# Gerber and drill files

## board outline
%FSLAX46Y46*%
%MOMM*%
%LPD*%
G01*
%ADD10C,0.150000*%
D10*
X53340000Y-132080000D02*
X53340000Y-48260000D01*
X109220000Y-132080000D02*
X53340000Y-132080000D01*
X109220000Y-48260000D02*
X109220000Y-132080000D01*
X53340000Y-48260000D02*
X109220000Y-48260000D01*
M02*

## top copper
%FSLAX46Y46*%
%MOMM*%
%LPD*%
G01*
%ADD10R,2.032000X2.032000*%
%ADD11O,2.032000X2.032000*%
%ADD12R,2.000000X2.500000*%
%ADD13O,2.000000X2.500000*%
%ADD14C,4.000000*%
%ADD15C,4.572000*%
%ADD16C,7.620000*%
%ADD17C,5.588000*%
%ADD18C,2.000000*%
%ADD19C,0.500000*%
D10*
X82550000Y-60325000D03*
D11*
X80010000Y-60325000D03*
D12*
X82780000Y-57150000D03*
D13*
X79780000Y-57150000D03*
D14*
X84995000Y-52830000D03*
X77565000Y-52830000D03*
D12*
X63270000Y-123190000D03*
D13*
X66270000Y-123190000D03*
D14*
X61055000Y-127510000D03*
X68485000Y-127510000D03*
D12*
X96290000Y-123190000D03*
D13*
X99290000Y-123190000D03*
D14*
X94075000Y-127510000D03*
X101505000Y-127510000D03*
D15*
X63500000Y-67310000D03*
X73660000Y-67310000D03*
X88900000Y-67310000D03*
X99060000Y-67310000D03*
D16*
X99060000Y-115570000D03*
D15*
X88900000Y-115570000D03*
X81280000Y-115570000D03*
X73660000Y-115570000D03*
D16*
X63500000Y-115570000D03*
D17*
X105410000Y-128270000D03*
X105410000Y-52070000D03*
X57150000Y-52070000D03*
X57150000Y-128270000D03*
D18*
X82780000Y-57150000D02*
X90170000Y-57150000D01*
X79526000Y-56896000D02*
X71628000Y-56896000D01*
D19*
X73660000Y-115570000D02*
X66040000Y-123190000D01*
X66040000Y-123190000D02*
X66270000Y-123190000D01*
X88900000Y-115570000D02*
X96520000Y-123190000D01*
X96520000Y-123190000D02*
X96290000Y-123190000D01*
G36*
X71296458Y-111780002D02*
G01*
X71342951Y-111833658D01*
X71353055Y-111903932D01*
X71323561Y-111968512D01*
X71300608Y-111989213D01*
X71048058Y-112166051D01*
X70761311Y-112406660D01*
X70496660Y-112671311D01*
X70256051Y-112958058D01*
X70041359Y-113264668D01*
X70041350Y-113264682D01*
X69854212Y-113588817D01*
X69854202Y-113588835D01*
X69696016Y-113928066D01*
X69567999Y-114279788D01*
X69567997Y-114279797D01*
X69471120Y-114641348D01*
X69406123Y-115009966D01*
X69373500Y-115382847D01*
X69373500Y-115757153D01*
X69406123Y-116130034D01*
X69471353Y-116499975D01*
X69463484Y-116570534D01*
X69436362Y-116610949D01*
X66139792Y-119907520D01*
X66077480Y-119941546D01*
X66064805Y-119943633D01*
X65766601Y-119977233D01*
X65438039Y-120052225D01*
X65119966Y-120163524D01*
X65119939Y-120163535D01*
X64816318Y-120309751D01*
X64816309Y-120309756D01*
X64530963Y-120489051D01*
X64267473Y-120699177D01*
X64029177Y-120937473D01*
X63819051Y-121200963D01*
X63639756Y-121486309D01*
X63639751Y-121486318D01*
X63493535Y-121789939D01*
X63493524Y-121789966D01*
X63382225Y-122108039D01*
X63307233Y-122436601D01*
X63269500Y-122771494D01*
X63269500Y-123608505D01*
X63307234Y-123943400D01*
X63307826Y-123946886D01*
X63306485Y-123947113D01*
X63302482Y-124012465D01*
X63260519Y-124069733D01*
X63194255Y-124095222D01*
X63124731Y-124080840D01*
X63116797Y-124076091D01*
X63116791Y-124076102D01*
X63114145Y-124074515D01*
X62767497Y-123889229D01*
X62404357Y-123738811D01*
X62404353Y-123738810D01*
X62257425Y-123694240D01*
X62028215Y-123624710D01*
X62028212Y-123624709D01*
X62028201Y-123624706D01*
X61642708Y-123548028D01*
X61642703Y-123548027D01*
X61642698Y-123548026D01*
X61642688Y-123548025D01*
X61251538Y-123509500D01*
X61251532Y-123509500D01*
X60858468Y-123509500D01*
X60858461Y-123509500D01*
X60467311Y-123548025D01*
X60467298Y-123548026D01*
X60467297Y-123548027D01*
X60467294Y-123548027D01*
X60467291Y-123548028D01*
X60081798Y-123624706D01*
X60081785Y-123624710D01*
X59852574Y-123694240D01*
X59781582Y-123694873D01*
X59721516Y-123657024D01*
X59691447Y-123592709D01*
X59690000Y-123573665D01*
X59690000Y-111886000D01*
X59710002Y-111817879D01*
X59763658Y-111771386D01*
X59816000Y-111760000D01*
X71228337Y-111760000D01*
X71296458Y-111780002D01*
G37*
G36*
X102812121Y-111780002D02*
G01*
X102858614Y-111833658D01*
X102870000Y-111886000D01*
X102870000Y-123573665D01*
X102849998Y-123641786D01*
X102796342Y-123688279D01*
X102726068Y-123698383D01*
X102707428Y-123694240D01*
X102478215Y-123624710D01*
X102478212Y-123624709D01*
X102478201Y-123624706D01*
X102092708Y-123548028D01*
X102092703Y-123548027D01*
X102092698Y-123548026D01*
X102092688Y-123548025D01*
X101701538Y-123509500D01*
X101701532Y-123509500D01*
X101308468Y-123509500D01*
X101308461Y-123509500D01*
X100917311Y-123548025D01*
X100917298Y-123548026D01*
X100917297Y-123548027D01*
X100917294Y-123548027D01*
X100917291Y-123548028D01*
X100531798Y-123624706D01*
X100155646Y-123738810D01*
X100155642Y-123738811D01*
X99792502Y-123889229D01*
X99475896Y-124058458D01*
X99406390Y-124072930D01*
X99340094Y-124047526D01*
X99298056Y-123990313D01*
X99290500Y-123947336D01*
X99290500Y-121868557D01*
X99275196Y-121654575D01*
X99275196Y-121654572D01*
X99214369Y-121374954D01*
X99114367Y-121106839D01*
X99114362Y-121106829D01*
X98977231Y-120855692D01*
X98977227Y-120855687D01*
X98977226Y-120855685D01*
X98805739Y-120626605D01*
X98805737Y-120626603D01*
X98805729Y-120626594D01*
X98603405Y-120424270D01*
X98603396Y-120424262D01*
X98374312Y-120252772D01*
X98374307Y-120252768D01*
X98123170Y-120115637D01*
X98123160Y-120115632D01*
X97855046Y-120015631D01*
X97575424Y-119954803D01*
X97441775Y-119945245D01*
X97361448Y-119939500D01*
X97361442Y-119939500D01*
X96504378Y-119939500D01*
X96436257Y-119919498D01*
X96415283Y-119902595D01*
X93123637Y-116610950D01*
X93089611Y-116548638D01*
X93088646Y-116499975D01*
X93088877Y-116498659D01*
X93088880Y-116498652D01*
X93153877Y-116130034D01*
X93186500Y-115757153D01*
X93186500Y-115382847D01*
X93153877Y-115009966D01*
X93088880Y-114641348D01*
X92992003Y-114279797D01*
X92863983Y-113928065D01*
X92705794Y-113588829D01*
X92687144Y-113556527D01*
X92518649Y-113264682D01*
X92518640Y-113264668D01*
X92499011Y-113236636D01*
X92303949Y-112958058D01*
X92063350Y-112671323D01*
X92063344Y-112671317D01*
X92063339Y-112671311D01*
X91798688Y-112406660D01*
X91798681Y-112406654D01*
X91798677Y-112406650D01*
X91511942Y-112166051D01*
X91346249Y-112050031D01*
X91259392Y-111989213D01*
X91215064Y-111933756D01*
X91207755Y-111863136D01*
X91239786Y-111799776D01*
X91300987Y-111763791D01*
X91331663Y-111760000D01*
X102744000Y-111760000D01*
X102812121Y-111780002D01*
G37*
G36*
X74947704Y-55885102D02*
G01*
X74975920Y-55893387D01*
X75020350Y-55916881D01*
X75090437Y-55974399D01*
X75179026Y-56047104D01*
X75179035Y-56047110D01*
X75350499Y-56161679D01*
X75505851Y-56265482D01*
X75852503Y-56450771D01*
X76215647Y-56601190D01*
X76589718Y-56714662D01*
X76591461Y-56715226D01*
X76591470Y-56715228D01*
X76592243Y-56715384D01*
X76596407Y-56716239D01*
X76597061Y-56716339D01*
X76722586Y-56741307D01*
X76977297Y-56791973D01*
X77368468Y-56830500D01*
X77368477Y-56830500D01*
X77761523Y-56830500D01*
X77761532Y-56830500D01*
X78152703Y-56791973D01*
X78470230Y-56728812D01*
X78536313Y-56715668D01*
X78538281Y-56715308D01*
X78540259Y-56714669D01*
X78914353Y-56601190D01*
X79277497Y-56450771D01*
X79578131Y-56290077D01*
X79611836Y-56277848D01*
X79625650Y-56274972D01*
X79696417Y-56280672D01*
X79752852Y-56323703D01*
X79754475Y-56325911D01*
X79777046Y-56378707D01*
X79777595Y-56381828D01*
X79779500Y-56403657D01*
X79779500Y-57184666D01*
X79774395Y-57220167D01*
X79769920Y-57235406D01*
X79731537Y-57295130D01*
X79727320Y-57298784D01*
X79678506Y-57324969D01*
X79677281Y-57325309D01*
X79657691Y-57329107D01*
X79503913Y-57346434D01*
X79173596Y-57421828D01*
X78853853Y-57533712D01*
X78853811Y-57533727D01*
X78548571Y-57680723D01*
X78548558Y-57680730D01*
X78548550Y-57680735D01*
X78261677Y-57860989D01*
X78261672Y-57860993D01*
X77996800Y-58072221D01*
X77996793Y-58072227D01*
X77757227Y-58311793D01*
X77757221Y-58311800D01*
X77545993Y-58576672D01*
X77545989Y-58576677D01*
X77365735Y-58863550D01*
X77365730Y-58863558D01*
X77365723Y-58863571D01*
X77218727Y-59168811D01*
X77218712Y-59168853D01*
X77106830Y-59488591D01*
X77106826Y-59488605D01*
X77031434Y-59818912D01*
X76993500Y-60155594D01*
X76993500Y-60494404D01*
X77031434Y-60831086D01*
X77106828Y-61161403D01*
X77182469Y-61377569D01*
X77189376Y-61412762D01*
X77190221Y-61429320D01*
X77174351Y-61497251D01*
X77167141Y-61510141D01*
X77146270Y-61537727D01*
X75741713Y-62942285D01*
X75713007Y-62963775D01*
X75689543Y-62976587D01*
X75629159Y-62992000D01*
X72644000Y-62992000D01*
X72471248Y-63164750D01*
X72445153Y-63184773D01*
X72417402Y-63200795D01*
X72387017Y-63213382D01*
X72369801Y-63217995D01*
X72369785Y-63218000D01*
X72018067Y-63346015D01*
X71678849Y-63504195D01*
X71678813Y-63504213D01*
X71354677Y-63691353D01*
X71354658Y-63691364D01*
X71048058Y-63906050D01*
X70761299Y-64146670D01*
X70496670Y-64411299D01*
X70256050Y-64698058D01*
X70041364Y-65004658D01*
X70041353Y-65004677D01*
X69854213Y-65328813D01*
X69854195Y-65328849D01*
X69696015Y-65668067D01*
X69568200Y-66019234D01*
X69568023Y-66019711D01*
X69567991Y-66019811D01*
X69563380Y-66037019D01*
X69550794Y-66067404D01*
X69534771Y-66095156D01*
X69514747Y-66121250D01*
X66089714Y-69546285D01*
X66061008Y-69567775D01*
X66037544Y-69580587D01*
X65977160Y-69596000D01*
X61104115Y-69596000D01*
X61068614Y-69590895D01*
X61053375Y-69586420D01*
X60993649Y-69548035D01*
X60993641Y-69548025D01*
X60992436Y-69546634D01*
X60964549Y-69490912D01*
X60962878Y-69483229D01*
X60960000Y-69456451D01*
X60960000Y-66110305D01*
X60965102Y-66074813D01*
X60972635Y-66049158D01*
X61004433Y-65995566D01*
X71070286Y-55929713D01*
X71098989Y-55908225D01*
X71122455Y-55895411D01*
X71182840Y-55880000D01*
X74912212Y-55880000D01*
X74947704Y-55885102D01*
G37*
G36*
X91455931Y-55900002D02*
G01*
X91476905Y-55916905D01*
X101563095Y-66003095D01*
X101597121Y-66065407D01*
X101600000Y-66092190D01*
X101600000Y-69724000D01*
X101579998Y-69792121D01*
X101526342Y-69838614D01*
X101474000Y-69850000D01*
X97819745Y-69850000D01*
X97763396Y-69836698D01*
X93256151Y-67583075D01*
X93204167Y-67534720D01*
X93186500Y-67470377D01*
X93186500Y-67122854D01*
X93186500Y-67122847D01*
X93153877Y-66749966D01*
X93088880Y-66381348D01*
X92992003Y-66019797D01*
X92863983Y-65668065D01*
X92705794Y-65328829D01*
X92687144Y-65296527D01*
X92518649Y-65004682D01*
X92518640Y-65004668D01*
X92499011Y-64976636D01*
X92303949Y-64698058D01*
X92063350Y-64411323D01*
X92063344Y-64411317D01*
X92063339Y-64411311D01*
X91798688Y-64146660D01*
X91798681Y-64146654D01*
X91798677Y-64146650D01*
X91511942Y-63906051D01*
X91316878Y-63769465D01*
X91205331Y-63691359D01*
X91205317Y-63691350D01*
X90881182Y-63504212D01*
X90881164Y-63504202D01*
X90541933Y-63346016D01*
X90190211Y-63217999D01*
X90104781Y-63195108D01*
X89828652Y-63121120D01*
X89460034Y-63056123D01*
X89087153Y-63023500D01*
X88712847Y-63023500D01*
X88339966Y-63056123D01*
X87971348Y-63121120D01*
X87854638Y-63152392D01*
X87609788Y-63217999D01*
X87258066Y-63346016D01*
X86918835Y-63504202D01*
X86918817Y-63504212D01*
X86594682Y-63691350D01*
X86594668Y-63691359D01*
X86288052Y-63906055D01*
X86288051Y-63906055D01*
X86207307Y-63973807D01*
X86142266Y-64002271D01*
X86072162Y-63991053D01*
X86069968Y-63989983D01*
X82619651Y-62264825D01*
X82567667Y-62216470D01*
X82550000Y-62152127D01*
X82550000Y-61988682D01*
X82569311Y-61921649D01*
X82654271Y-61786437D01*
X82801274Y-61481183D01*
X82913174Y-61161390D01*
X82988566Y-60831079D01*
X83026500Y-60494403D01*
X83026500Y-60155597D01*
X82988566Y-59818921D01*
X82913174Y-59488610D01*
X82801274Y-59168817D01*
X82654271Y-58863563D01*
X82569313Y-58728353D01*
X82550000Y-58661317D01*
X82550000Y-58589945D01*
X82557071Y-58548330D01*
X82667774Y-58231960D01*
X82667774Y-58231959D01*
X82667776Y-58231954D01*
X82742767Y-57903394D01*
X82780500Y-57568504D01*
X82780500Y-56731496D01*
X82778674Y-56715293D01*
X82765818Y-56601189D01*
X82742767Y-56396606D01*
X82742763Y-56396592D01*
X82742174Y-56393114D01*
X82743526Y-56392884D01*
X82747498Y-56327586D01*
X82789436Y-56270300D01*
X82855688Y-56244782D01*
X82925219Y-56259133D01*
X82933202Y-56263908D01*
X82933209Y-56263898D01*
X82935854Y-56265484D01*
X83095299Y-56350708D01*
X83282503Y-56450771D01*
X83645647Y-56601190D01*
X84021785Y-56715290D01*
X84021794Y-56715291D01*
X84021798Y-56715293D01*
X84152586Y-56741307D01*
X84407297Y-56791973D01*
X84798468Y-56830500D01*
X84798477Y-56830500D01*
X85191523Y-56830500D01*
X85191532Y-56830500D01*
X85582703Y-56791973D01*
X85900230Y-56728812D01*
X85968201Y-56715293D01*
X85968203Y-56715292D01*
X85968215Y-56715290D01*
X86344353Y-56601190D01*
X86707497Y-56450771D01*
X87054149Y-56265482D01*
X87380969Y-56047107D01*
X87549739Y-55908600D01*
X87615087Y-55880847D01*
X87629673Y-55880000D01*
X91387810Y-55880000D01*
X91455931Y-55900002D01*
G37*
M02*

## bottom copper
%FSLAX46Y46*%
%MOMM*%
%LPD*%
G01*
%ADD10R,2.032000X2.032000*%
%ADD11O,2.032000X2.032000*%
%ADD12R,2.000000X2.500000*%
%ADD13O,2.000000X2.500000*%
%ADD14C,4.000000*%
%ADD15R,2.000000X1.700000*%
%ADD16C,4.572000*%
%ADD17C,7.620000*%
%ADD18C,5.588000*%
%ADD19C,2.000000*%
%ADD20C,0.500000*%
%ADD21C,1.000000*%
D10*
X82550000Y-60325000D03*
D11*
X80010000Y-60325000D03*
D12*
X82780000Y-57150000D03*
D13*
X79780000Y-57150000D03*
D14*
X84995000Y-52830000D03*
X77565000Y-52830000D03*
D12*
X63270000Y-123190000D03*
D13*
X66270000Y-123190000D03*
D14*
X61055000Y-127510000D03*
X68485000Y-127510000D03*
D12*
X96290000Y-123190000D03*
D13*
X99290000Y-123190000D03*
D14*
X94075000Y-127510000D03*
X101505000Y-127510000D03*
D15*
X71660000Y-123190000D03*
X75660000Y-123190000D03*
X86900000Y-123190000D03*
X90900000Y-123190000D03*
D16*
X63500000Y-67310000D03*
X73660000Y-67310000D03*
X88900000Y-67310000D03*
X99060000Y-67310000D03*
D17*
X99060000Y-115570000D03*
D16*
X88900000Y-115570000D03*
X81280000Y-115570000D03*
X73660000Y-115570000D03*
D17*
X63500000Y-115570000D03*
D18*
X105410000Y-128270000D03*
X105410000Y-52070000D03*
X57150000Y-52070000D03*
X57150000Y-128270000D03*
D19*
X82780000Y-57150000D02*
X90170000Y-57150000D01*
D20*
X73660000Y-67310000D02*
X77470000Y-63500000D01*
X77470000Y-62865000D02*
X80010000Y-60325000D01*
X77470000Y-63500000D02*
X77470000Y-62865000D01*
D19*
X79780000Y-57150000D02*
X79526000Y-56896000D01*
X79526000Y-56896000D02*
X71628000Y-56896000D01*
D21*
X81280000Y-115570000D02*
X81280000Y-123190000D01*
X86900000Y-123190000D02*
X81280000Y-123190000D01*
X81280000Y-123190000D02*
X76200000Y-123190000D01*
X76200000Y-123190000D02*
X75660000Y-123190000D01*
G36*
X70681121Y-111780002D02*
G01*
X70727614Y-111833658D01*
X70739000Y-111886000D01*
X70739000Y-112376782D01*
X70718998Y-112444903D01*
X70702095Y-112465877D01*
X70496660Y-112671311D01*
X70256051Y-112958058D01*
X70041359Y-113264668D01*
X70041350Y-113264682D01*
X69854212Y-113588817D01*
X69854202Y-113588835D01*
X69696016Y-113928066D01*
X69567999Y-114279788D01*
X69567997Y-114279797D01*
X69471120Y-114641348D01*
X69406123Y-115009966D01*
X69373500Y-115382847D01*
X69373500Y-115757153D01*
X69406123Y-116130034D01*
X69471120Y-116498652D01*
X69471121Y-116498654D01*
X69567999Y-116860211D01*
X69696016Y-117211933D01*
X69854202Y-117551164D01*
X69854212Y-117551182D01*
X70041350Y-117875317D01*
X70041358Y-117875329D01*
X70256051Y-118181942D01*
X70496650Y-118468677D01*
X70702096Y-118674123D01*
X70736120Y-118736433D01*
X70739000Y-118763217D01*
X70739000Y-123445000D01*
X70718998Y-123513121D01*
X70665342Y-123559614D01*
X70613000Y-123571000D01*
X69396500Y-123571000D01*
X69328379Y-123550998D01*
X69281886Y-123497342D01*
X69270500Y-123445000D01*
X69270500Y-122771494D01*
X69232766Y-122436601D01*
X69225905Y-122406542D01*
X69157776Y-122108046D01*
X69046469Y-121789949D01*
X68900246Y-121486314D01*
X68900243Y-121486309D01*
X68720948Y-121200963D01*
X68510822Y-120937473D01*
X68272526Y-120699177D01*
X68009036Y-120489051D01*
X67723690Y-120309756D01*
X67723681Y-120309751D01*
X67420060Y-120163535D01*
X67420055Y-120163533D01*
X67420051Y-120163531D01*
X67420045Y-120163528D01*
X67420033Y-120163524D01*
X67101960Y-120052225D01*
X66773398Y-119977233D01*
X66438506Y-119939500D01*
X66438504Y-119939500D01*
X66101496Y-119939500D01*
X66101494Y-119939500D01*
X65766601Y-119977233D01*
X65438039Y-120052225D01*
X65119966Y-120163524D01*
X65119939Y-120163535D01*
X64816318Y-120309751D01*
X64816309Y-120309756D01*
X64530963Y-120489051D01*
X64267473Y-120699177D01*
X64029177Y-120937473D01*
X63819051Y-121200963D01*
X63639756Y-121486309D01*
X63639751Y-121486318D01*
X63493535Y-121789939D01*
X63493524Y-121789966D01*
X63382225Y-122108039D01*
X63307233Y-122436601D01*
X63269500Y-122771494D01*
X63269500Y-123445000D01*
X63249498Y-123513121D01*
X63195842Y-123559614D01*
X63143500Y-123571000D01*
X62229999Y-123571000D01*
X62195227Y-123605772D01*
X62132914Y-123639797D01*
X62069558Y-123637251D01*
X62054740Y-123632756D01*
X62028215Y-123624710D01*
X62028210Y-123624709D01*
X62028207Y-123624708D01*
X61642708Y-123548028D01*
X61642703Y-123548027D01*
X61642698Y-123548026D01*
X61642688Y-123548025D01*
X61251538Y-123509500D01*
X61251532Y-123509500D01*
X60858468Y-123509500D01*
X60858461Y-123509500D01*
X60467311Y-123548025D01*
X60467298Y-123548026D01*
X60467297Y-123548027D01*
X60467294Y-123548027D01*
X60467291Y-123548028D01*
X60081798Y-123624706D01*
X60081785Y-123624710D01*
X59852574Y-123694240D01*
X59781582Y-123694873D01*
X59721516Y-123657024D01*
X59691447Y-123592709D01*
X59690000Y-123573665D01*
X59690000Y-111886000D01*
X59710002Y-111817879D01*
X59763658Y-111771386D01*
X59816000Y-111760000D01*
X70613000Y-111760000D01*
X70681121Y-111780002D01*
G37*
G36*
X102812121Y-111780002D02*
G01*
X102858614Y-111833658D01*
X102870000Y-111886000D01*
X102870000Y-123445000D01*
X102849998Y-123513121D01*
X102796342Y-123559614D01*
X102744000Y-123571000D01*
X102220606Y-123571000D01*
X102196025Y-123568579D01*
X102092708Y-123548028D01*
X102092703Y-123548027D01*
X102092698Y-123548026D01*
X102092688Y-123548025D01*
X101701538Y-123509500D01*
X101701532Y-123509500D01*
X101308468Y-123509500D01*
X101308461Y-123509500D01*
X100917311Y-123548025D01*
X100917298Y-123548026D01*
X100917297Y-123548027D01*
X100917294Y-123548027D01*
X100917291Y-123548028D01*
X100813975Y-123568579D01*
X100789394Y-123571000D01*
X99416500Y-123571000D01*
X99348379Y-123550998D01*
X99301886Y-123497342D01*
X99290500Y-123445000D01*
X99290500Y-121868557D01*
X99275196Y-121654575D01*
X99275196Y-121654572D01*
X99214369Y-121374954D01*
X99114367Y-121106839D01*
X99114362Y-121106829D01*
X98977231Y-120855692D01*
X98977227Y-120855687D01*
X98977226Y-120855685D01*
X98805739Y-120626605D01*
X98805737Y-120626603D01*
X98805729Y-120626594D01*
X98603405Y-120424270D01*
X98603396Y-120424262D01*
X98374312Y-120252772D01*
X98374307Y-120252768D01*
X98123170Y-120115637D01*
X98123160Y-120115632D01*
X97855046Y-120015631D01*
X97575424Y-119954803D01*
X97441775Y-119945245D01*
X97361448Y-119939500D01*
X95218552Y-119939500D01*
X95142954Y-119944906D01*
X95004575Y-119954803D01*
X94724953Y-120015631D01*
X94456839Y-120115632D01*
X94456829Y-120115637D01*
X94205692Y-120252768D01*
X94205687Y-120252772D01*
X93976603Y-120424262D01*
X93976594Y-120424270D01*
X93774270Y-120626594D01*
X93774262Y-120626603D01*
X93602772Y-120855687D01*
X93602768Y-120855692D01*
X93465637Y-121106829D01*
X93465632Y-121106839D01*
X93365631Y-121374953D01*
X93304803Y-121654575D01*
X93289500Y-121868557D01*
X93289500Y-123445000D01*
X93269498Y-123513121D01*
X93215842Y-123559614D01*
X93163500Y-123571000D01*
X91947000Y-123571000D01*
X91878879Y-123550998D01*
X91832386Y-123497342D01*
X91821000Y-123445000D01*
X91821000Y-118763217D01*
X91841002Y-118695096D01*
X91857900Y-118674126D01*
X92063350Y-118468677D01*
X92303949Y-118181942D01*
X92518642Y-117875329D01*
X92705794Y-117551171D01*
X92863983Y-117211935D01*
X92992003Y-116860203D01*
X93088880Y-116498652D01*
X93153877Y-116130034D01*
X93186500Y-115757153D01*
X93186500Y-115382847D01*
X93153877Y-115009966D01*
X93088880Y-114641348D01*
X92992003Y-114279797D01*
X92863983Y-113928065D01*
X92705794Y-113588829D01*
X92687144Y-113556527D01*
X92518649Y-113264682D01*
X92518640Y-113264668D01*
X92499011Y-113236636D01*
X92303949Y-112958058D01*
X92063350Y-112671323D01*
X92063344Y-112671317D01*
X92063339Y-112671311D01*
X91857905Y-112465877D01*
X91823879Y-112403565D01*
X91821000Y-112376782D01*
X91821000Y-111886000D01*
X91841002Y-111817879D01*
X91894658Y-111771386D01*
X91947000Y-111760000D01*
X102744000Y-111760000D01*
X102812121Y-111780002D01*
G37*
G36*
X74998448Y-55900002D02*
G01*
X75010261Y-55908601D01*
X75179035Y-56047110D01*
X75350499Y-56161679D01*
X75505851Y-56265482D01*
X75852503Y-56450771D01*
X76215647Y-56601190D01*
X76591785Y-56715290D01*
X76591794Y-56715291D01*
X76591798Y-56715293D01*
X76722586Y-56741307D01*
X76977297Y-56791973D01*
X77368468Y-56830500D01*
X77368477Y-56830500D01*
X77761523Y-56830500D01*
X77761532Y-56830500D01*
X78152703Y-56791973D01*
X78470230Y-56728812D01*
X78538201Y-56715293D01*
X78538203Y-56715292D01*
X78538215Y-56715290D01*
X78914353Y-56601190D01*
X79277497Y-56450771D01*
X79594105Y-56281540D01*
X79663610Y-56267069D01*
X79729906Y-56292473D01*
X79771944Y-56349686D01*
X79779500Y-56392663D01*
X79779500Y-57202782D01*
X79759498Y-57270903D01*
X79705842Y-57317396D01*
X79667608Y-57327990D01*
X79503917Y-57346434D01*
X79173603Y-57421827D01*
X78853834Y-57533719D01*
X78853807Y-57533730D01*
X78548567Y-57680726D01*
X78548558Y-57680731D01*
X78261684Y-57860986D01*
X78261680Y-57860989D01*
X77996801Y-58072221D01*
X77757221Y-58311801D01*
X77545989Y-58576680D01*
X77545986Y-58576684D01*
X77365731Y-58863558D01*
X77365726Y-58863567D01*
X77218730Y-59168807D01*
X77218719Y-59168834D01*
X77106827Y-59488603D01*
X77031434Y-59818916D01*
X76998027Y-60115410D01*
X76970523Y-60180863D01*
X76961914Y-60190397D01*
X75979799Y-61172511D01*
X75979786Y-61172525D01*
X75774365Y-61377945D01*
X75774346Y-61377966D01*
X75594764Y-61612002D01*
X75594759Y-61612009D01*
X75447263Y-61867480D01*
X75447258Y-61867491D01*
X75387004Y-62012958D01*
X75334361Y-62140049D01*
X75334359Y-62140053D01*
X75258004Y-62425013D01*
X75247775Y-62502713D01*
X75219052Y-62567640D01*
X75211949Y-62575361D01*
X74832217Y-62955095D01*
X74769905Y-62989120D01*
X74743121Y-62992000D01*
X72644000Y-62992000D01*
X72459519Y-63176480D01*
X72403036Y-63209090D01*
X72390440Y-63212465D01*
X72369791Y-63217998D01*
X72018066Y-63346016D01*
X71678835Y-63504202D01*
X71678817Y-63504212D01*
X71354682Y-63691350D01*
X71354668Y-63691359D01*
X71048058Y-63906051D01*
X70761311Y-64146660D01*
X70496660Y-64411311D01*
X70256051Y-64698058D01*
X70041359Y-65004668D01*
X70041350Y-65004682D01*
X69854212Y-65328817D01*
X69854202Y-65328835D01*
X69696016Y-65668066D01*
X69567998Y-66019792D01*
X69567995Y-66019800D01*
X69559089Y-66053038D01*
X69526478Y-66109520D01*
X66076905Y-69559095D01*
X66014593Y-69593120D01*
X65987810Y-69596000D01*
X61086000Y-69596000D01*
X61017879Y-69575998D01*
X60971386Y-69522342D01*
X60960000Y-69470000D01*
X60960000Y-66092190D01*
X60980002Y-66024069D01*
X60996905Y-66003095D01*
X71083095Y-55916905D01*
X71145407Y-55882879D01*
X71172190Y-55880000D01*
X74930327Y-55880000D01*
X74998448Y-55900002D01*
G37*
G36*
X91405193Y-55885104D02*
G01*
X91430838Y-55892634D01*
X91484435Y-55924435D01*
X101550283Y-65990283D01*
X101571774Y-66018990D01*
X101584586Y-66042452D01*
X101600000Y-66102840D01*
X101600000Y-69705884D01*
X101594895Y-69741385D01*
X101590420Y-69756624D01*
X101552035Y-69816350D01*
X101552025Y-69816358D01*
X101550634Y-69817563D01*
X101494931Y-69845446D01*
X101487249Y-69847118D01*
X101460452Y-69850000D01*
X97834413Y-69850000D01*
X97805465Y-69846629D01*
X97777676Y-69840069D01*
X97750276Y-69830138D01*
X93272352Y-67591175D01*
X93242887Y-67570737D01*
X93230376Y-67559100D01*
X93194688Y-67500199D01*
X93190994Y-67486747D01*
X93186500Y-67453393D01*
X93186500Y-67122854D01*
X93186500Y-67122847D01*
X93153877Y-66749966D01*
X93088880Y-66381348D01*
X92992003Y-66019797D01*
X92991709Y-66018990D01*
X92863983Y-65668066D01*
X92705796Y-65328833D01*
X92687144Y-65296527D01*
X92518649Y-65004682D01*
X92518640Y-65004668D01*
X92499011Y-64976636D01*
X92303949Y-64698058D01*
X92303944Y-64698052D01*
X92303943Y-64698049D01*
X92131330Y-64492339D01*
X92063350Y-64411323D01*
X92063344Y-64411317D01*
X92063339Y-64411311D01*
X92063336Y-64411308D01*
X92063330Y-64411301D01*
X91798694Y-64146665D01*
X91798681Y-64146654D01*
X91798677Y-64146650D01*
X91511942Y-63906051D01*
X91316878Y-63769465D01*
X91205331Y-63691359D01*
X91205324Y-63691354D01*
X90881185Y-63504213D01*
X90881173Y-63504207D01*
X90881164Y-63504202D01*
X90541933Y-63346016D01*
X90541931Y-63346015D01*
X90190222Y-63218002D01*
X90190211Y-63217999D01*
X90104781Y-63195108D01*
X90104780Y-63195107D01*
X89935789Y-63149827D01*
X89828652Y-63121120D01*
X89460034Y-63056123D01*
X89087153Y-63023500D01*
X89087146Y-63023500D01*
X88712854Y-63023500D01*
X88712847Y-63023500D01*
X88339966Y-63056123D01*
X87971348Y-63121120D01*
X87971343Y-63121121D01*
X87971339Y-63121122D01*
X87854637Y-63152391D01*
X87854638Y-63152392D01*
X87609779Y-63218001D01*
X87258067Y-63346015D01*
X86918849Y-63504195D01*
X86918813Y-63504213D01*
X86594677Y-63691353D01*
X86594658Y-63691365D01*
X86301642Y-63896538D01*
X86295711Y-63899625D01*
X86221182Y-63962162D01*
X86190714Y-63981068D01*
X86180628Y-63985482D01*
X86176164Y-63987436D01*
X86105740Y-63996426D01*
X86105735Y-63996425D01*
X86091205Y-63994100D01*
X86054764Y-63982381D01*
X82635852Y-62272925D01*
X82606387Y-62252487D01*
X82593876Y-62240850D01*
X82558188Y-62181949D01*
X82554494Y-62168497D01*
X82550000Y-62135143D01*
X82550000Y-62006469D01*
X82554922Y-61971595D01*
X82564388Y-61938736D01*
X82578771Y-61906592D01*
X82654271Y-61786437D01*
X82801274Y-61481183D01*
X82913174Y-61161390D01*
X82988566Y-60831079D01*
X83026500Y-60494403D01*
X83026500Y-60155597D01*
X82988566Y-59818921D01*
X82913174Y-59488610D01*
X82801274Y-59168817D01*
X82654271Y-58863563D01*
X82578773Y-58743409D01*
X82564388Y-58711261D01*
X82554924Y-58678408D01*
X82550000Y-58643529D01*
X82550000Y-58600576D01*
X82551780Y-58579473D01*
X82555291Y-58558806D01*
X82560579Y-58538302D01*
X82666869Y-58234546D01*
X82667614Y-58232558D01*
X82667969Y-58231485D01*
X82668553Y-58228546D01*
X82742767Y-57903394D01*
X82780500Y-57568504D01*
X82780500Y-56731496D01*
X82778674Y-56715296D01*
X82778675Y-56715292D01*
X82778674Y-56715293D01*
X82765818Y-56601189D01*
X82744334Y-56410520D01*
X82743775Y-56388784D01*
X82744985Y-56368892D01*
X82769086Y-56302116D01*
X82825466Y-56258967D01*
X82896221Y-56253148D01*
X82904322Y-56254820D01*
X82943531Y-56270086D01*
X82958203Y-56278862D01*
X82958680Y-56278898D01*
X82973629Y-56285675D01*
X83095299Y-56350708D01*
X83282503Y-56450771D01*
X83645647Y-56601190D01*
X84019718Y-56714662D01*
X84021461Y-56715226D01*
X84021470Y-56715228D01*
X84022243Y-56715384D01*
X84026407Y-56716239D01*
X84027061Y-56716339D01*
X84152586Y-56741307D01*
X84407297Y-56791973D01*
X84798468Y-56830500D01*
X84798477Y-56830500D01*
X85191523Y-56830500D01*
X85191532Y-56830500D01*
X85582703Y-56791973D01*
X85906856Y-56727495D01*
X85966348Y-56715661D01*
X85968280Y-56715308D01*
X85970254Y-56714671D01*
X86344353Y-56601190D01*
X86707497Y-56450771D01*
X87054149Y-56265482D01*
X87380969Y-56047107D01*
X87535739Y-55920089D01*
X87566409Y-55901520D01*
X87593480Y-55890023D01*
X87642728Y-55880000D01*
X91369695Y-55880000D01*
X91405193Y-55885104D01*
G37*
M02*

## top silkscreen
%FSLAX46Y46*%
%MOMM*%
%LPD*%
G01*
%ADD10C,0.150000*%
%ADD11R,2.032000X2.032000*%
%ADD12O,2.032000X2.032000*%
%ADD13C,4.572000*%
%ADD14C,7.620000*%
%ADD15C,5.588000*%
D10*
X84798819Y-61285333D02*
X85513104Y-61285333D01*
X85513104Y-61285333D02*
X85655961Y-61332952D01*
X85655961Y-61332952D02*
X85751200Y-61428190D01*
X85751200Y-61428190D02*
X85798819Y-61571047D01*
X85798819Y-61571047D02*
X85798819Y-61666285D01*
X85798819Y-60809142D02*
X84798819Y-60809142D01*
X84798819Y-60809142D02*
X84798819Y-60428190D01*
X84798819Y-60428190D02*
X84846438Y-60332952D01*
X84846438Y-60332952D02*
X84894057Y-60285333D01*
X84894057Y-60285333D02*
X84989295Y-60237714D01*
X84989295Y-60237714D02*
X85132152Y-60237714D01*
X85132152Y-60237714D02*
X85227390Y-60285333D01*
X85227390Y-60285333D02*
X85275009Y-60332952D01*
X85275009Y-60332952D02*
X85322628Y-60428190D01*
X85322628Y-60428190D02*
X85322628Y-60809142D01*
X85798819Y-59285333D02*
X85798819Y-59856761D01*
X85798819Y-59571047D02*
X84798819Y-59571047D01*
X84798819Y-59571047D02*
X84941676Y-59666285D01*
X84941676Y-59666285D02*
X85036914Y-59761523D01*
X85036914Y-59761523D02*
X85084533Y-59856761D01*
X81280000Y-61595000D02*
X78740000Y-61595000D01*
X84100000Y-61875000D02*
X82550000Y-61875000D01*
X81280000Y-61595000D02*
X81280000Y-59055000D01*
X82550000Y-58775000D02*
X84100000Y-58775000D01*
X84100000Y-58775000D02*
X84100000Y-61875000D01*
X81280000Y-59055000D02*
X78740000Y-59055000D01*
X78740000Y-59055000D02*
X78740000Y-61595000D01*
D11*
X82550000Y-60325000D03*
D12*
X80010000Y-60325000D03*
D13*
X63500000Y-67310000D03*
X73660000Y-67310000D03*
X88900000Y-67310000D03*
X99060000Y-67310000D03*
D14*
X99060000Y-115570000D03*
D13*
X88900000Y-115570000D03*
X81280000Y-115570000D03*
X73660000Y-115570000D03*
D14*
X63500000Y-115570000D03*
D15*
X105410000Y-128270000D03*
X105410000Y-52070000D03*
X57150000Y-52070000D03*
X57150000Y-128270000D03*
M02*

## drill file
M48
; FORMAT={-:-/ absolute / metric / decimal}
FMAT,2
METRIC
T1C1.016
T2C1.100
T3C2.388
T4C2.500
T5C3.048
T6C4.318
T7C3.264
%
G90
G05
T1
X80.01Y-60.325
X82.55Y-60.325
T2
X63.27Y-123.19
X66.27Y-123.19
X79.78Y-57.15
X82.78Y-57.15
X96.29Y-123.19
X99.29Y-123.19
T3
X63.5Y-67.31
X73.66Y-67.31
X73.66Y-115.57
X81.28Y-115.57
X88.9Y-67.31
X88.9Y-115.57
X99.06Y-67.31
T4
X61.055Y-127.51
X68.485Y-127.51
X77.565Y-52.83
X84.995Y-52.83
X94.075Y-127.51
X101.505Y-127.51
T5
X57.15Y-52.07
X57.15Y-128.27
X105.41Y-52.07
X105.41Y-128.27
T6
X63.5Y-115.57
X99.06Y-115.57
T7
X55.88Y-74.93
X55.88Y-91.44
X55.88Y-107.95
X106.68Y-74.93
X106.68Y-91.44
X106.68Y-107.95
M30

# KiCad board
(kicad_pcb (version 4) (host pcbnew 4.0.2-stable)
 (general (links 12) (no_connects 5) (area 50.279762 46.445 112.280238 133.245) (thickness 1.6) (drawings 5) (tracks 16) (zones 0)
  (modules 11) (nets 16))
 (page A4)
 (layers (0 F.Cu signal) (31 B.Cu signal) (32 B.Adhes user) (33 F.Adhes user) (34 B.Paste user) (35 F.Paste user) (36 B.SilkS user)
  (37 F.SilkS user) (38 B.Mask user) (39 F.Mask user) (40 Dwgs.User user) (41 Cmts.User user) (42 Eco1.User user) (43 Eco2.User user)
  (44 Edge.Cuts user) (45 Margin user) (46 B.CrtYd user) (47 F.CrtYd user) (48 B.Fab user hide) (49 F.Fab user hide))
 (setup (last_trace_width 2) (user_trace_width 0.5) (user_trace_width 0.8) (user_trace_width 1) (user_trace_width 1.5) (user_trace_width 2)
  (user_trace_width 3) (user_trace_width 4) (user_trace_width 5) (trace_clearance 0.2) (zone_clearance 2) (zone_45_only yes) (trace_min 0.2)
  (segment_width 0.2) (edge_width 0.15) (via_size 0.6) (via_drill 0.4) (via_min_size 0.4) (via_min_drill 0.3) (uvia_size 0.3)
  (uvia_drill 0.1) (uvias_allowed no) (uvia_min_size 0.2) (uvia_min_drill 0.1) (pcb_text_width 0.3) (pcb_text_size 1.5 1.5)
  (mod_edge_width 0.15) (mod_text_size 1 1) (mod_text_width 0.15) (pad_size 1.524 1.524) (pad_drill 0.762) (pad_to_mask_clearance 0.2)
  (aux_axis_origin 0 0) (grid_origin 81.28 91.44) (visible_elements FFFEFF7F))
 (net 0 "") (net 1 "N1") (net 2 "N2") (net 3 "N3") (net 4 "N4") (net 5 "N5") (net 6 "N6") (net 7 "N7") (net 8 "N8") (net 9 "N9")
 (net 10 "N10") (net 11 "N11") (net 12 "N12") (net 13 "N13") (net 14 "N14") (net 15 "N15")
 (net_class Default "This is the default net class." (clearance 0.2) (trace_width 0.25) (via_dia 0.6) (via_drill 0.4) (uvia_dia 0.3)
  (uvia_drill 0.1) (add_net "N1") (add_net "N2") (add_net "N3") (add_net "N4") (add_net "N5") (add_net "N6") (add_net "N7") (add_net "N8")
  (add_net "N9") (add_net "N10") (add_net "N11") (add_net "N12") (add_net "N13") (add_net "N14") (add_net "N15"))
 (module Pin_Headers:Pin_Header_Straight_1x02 (layer F.Cu) (at 82.55 60.325 270)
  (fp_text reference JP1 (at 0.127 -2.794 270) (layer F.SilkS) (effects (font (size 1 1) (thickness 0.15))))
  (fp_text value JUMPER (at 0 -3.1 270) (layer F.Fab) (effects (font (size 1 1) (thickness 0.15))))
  (fp_line (start 1.27 1.27) (end 1.27 3.81) (layer F.SilkS) (width 0.15))
  (fp_line (start 1.55 -1.55) (end 1.55 0) (layer F.SilkS) (width 0.15))
  (fp_line (start 1.27 1.27) (end -1.27 1.27) (layer F.SilkS) (width 0.15))
  (fp_line (start -1.55 0) (end -1.55 -1.55) (layer F.SilkS) (width 0.15))
  (fp_line (start -1.55 -1.55) (end 1.55 -1.55) (layer F.SilkS) (width 0.15))
  (fp_line (start -1.27 1.27) (end -1.27 3.81) (layer F.SilkS) (width 0.15))
  (fp_line (start -1.27 3.81) (end 1.27 3.81) (layer F.SilkS) (width 0.15))
  (pad 1 thru_hole rect (at 0 0 270) (size 2.032 2.032) (drill 1.016) (layers *.Cu *.Mask F.SilkS) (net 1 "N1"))
  (pad 2 thru_hole oval (at 0 2.54 270) (size 2.032 2.032) (drill 1.016) (layers *.Cu *.Mask F.SilkS) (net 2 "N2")))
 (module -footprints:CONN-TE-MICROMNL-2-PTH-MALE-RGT (layer B.Cu) (at 81.28 57.15)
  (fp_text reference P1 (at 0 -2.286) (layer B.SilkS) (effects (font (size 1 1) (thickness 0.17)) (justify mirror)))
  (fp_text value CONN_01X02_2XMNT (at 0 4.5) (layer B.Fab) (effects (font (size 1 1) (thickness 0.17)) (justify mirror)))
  (pad 1 thru_hole rect (at 1.5 0) (size 2 2.5) (drill 1.1) (layers *.Cu *.Mask B.SilkS) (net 1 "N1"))
  (pad 2 thru_hole oval (at -1.5 0) (size 2 2.5) (drill 1.1) (layers *.Cu *.Mask B.SilkS) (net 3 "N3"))
  (pad M1 thru_hole circle (at 3.715 -4.32) (size 4 4) (drill 2.5) (layers *.Cu *.Mask B.SilkS) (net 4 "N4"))
  (pad M2 thru_hole circle (at -3.715 -4.32) (size 4 4) (drill 2.5) (layers *.Cu *.Mask B.SilkS) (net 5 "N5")))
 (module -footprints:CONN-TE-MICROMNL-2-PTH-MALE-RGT (layer B.Cu) (at 64.77 123.19 180)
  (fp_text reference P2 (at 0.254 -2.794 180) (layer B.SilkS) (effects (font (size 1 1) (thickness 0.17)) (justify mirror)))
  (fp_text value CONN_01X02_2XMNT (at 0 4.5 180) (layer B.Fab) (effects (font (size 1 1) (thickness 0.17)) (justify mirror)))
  (pad 1 thru_hole rect (at 1.5 0 180) (size 2 2.5) (drill 1.1) (layers *.Cu *.Mask B.SilkS) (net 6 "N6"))
  (pad 2 thru_hole oval (at -1.5 0 180) (size 2 2.5) (drill 1.1) (layers *.Cu *.Mask B.SilkS) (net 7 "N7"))
  (pad M1 thru_hole circle (at 3.715 -4.32 180) (size 4 4) (drill 2.5) (layers *.Cu *.Mask B.SilkS) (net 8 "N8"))
  (pad M2 thru_hole circle (at -3.715 -4.32 180) (size 4 4) (drill 2.5) (layers *.Cu *.Mask B.SilkS) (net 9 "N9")))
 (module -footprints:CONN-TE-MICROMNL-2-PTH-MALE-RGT (layer B.Cu) (at 97.79 123.19 180)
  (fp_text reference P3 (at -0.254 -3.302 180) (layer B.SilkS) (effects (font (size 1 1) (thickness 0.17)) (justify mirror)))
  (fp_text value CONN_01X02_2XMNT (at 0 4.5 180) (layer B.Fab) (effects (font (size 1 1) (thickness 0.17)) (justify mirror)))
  (pad 1 thru_hole rect (at 1.5 0 180) (size 2 2.5) (drill 1.1) (layers *.Cu *.Mask B.SilkS) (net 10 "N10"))
  (pad 2 thru_hole oval (at -1.5 0 180) (size 2 2.5) (drill 1.1) (layers *.Cu *.Mask B.SilkS) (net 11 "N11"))
  (pad M1 thru_hole circle (at 3.715 -4.32 180) (size 4 4) (drill 2.5) (layers *.Cu *.Mask B.SilkS) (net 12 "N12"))
  (pad M2 thru_hole circle (at -3.715 -4.32 180) (size 4 4) (drill 2.5) (layers *.Cu *.Mask B.SilkS) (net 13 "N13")))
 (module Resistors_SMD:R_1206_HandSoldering (layer B.Cu) (at 73.66 123.19)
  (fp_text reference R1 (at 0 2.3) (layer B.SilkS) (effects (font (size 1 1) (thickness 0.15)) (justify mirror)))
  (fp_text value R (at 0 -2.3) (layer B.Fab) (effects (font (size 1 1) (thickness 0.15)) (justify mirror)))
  (pad 1 smd rect (at -2 0) (size 2 1.7) (layers B.Cu B.Paste B.Mask) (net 6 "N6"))
  (pad 2 smd rect (at 2 0) (size 2 1.7) (layers B.Cu B.Paste B.Mask) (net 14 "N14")))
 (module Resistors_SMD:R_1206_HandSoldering (layer B.Cu) (at 88.9 123.19)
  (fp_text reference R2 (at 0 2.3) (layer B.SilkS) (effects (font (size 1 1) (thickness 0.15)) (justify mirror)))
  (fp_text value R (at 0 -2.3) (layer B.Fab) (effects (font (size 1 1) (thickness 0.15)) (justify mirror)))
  (pad 1 smd rect (at -2 0) (size 2 1.7) (layers B.Cu B.Paste B.Mask) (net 14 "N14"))
  (pad 2 smd rect (at 2 0) (size 2 1.7) (layers B.Cu B.Paste B.Mask) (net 11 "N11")))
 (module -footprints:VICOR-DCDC (layer F.Cu) (at 81.28 91.44)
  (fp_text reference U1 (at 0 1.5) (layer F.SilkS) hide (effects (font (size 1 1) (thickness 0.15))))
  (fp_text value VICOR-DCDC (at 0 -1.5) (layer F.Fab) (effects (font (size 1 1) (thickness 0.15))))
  (pad 1 thru_hole circle (at -17.78 -24.13) (size 4.572 4.572) (drill 2.3876) (layers *.Cu *.Mask F.SilkS) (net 3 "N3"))
  (pad 2 thru_hole circle (at -7.62 -24.13) (size 4.572 4.572) (drill 2.3876) (layers *.Cu *.Mask F.SilkS) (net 2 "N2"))
  (pad 3 thru_hole circle (at 7.62 -24.13) (size 4.572 4.572) (drill 2.3876) (layers *.Cu *.Mask F.SilkS) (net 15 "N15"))
  (pad 4 thru_hole circle (at 17.78 -24.13) (size 4.572 4.572) (drill 2.3876) (layers *.Cu *.Mask F.SilkS) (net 1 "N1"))
  (pad 5 thru_hole circle (at 17.78 24.13) (size 7.62 7.62) (drill 4.318) (layers *.Cu *.Mask F.SilkS) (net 11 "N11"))
  (pad 6 thru_hole circle (at 7.62 24.13) (size 4.572 4.572) (drill 2.3876) (layers *.Cu *.Mask F.SilkS) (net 10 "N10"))
  (pad 7 thru_hole circle (at 0 24.13) (size 4.572 4.572) (drill 2.3876) (layers *.Cu *.Mask F.SilkS) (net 14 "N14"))
  (pad 8 thru_hole circle (at -7.62 24.13) (size 4.572 4.572) (drill 2.3876) (layers *.Cu *.Mask F.SilkS) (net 7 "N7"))
  (pad 9 thru_hole circle (at -17.78 24.13) (size 7.62 7.62) (drill 4.318) (layers *.Cu *.Mask F.SilkS) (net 6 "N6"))
  (pad "" np_thru_hole circle (at -25.4 0) (size 3.2639 3.2639) (drill 3.2639) (layers *.Cu))
  (pad "" np_thru_hole circle (at 25.4 0) (size 3.2639 3.2639) (drill 3.2639) (layers *.Cu))
  (pad "" np_thru_hole circle (at 25.4 -16.51) (size 3.2639 3.2639) (drill 3.2639) (layers *.Cu))
  (pad "" np_thru_hole circle (at 25.4 16.51) (size 3.2639 3.2639) (drill 3.2639) (layers *.Cu))
  (pad "" np_thru_hole circle (at -25.4 16.51) (size 3.2639 3.2639) (drill 3.2639) (layers *.Cu))
  (pad "" np_thru_hole circle (at -25.4 -16.51) (size 3.2639 3.2639) (drill 3.2639) (layers *.Cu)))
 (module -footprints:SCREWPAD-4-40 (layer F.Cu) (at 105.41 128.27)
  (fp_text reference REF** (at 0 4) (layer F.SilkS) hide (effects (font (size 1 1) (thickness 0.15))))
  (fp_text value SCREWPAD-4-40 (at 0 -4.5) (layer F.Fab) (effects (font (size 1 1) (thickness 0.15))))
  (pad 1 thru_hole circle (at 0 0) (size 5.588 5.588) (drill 3.048) (layers *.Cu *.Mask F.SilkS)))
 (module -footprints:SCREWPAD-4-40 (layer F.Cu) (at 105.41 52.07)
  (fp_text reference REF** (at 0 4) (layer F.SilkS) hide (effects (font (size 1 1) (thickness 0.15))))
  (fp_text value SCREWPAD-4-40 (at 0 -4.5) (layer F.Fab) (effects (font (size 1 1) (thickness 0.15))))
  (pad 1 thru_hole circle (at 0 0) (size 5.588 5.588) (drill 3.048) (layers *.Cu *.Mask F.SilkS)))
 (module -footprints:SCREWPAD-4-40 (layer F.Cu) (at 57.15 52.07)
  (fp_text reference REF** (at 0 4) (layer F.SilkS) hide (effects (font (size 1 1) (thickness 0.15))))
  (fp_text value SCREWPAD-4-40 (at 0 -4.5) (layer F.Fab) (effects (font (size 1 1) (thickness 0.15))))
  (pad 1 thru_hole circle (at 0 0) (size 5.588 5.588) (drill 3.048) (layers *.Cu *.Mask F.SilkS)))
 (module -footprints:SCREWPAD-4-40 (layer F.Cu) (at 57.15 128.27)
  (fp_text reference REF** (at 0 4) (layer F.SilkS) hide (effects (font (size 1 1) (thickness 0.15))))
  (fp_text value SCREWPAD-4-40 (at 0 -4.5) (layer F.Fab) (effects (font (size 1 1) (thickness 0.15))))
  (pad 1 thru_hole circle (at 0 0) (size 5.588 5.588) (drill 3.048) (layers *.Cu *.Mask F.SilkS)))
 (gr_line (start 53.34 132.08) (end 53.34 48.26) (angle 90) (layer Edge.Cuts) (width 0.15))
 (gr_line (start 109.22 132.08) (end 53.34 132.08) (angle 90) (layer Edge.Cuts) (width 0.15))
 (gr_line (start 109.22 48.26) (end 109.22 132.08) (angle 90) (layer Edge.Cuts) (width 0.15))
 (gr_line (start 53.34 48.26) (end 109.22 48.26) (angle 90) (layer Edge.Cuts) (width 0.15))
 (segment (start 82.78 57.15) (end 90.17 57.15) (width 2) (layer F.Cu) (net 1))
 (segment (start 82.78 57.15) (end 90.17 57.15) (width 2) (layer B.Cu) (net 1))
 (segment (start 73.66 67.31) (end 77.47 63.5) (width 0.5) (layer B.Cu) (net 2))
 (segment (start 77.47 62.865) (end 80.01 60.325) (width 0.5) (layer B.Cu) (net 2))
 (segment (start 77.47 63.5) (end 77.47 62.865) (width 0.5) (layer B.Cu) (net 2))
 (segment (start 79.78 57.15) (end 79.526 56.896) (width 2) (layer B.Cu) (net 3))
 (segment (start 79.526 56.896) (end 71.628 56.896) (width 2) (layer B.Cu) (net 3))
 (segment (start 79.526 56.896) (end 71.628 56.896) (width 2) (layer F.Cu) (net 3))
 (segment (start 73.66 115.57) (end 66.04 123.19) (width 0.5) (layer F.Cu) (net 7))
 (segment (start 66.04 123.19) (end 66.27 123.19) (width 0.5) (layer F.Cu) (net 7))
 (segment (start 81.28 115.57) (end 81.28 123.19) (width 1) (layer B.Cu) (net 14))
 (segment (start 86.9 123.19) (end 81.28 123.19) (width 1) (layer B.Cu) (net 14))
 (segment (start 81.28 123.19) (end 76.2 123.19) (width 1) (layer B.Cu) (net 14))
 (segment (start 76.2 123.19) (end 75.66 123.19) (width 1) (layer B.Cu) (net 14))
 (segment (start 88.9 115.57) (end 96.52 123.19) (width 0.5) (layer F.Cu) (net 10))
 (segment (start 96.52 123.19) (end 96.29 123.19) (width 0.5) (layer F.Cu) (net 10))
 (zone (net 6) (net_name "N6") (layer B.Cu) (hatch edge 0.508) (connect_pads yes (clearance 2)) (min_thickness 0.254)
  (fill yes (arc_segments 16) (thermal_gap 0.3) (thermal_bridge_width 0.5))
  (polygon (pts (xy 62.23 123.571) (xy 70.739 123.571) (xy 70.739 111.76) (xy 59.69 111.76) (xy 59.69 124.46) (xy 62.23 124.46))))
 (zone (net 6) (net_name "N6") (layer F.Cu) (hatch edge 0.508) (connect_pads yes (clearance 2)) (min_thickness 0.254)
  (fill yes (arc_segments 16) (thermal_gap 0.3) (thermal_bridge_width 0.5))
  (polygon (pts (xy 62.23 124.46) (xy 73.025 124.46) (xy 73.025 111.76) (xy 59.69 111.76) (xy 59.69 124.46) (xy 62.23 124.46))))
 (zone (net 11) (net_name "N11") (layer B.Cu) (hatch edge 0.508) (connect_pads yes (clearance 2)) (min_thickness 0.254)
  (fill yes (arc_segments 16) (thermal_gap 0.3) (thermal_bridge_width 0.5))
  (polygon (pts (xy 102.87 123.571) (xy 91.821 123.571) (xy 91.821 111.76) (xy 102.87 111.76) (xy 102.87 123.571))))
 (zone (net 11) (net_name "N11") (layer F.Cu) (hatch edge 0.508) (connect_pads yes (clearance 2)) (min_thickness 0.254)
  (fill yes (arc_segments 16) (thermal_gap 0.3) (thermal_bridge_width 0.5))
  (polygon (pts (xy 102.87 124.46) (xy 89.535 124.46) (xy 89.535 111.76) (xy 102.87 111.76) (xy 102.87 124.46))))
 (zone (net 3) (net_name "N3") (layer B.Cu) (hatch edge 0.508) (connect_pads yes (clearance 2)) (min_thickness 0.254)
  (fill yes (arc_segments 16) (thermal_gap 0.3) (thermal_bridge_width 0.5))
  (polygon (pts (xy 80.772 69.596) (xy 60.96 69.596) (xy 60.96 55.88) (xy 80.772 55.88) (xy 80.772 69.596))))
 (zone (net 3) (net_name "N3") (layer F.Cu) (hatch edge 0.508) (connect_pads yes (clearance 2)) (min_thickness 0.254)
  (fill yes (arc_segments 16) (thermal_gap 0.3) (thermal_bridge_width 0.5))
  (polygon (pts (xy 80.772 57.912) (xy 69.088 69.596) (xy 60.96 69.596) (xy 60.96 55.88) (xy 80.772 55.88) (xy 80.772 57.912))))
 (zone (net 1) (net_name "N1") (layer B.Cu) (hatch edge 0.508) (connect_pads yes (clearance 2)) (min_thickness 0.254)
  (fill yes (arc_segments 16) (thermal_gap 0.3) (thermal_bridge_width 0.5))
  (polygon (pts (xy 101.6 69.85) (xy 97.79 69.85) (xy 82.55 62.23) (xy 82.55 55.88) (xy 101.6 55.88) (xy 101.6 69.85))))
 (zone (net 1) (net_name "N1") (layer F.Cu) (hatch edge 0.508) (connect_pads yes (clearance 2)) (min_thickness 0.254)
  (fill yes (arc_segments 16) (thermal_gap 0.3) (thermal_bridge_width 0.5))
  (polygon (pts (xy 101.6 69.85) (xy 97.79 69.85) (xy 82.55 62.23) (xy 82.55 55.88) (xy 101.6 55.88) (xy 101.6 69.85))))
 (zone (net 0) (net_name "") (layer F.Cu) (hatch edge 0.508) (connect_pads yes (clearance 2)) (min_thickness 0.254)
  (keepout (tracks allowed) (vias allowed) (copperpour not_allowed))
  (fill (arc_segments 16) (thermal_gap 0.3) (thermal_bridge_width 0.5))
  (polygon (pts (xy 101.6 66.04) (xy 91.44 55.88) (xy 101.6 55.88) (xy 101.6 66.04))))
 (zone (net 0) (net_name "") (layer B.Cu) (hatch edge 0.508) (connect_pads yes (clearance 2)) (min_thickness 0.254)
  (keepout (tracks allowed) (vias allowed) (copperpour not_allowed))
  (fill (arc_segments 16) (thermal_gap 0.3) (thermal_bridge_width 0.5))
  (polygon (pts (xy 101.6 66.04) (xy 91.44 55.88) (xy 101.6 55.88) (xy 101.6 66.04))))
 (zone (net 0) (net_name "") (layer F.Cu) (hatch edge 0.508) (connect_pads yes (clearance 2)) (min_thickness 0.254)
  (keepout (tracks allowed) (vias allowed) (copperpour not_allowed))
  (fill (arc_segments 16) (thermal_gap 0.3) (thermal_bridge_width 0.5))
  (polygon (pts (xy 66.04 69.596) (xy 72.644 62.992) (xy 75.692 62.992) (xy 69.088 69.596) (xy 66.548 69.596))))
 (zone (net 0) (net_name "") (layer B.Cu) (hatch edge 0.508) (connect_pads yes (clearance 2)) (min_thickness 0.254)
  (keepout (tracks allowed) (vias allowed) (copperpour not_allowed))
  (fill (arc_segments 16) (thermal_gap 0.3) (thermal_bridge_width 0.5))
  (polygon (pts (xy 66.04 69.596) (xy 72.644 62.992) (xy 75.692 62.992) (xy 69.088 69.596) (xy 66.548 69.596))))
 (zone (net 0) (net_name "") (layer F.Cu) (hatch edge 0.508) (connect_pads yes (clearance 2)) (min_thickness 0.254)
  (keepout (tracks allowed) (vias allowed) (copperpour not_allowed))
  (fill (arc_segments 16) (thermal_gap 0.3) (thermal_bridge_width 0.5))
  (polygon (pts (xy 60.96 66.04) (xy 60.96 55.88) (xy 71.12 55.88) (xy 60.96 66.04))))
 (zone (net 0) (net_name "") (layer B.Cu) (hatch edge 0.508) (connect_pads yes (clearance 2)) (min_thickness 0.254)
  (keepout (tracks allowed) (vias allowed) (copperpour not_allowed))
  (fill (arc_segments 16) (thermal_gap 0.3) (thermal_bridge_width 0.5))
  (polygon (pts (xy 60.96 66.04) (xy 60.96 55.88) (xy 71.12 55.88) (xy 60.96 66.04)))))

